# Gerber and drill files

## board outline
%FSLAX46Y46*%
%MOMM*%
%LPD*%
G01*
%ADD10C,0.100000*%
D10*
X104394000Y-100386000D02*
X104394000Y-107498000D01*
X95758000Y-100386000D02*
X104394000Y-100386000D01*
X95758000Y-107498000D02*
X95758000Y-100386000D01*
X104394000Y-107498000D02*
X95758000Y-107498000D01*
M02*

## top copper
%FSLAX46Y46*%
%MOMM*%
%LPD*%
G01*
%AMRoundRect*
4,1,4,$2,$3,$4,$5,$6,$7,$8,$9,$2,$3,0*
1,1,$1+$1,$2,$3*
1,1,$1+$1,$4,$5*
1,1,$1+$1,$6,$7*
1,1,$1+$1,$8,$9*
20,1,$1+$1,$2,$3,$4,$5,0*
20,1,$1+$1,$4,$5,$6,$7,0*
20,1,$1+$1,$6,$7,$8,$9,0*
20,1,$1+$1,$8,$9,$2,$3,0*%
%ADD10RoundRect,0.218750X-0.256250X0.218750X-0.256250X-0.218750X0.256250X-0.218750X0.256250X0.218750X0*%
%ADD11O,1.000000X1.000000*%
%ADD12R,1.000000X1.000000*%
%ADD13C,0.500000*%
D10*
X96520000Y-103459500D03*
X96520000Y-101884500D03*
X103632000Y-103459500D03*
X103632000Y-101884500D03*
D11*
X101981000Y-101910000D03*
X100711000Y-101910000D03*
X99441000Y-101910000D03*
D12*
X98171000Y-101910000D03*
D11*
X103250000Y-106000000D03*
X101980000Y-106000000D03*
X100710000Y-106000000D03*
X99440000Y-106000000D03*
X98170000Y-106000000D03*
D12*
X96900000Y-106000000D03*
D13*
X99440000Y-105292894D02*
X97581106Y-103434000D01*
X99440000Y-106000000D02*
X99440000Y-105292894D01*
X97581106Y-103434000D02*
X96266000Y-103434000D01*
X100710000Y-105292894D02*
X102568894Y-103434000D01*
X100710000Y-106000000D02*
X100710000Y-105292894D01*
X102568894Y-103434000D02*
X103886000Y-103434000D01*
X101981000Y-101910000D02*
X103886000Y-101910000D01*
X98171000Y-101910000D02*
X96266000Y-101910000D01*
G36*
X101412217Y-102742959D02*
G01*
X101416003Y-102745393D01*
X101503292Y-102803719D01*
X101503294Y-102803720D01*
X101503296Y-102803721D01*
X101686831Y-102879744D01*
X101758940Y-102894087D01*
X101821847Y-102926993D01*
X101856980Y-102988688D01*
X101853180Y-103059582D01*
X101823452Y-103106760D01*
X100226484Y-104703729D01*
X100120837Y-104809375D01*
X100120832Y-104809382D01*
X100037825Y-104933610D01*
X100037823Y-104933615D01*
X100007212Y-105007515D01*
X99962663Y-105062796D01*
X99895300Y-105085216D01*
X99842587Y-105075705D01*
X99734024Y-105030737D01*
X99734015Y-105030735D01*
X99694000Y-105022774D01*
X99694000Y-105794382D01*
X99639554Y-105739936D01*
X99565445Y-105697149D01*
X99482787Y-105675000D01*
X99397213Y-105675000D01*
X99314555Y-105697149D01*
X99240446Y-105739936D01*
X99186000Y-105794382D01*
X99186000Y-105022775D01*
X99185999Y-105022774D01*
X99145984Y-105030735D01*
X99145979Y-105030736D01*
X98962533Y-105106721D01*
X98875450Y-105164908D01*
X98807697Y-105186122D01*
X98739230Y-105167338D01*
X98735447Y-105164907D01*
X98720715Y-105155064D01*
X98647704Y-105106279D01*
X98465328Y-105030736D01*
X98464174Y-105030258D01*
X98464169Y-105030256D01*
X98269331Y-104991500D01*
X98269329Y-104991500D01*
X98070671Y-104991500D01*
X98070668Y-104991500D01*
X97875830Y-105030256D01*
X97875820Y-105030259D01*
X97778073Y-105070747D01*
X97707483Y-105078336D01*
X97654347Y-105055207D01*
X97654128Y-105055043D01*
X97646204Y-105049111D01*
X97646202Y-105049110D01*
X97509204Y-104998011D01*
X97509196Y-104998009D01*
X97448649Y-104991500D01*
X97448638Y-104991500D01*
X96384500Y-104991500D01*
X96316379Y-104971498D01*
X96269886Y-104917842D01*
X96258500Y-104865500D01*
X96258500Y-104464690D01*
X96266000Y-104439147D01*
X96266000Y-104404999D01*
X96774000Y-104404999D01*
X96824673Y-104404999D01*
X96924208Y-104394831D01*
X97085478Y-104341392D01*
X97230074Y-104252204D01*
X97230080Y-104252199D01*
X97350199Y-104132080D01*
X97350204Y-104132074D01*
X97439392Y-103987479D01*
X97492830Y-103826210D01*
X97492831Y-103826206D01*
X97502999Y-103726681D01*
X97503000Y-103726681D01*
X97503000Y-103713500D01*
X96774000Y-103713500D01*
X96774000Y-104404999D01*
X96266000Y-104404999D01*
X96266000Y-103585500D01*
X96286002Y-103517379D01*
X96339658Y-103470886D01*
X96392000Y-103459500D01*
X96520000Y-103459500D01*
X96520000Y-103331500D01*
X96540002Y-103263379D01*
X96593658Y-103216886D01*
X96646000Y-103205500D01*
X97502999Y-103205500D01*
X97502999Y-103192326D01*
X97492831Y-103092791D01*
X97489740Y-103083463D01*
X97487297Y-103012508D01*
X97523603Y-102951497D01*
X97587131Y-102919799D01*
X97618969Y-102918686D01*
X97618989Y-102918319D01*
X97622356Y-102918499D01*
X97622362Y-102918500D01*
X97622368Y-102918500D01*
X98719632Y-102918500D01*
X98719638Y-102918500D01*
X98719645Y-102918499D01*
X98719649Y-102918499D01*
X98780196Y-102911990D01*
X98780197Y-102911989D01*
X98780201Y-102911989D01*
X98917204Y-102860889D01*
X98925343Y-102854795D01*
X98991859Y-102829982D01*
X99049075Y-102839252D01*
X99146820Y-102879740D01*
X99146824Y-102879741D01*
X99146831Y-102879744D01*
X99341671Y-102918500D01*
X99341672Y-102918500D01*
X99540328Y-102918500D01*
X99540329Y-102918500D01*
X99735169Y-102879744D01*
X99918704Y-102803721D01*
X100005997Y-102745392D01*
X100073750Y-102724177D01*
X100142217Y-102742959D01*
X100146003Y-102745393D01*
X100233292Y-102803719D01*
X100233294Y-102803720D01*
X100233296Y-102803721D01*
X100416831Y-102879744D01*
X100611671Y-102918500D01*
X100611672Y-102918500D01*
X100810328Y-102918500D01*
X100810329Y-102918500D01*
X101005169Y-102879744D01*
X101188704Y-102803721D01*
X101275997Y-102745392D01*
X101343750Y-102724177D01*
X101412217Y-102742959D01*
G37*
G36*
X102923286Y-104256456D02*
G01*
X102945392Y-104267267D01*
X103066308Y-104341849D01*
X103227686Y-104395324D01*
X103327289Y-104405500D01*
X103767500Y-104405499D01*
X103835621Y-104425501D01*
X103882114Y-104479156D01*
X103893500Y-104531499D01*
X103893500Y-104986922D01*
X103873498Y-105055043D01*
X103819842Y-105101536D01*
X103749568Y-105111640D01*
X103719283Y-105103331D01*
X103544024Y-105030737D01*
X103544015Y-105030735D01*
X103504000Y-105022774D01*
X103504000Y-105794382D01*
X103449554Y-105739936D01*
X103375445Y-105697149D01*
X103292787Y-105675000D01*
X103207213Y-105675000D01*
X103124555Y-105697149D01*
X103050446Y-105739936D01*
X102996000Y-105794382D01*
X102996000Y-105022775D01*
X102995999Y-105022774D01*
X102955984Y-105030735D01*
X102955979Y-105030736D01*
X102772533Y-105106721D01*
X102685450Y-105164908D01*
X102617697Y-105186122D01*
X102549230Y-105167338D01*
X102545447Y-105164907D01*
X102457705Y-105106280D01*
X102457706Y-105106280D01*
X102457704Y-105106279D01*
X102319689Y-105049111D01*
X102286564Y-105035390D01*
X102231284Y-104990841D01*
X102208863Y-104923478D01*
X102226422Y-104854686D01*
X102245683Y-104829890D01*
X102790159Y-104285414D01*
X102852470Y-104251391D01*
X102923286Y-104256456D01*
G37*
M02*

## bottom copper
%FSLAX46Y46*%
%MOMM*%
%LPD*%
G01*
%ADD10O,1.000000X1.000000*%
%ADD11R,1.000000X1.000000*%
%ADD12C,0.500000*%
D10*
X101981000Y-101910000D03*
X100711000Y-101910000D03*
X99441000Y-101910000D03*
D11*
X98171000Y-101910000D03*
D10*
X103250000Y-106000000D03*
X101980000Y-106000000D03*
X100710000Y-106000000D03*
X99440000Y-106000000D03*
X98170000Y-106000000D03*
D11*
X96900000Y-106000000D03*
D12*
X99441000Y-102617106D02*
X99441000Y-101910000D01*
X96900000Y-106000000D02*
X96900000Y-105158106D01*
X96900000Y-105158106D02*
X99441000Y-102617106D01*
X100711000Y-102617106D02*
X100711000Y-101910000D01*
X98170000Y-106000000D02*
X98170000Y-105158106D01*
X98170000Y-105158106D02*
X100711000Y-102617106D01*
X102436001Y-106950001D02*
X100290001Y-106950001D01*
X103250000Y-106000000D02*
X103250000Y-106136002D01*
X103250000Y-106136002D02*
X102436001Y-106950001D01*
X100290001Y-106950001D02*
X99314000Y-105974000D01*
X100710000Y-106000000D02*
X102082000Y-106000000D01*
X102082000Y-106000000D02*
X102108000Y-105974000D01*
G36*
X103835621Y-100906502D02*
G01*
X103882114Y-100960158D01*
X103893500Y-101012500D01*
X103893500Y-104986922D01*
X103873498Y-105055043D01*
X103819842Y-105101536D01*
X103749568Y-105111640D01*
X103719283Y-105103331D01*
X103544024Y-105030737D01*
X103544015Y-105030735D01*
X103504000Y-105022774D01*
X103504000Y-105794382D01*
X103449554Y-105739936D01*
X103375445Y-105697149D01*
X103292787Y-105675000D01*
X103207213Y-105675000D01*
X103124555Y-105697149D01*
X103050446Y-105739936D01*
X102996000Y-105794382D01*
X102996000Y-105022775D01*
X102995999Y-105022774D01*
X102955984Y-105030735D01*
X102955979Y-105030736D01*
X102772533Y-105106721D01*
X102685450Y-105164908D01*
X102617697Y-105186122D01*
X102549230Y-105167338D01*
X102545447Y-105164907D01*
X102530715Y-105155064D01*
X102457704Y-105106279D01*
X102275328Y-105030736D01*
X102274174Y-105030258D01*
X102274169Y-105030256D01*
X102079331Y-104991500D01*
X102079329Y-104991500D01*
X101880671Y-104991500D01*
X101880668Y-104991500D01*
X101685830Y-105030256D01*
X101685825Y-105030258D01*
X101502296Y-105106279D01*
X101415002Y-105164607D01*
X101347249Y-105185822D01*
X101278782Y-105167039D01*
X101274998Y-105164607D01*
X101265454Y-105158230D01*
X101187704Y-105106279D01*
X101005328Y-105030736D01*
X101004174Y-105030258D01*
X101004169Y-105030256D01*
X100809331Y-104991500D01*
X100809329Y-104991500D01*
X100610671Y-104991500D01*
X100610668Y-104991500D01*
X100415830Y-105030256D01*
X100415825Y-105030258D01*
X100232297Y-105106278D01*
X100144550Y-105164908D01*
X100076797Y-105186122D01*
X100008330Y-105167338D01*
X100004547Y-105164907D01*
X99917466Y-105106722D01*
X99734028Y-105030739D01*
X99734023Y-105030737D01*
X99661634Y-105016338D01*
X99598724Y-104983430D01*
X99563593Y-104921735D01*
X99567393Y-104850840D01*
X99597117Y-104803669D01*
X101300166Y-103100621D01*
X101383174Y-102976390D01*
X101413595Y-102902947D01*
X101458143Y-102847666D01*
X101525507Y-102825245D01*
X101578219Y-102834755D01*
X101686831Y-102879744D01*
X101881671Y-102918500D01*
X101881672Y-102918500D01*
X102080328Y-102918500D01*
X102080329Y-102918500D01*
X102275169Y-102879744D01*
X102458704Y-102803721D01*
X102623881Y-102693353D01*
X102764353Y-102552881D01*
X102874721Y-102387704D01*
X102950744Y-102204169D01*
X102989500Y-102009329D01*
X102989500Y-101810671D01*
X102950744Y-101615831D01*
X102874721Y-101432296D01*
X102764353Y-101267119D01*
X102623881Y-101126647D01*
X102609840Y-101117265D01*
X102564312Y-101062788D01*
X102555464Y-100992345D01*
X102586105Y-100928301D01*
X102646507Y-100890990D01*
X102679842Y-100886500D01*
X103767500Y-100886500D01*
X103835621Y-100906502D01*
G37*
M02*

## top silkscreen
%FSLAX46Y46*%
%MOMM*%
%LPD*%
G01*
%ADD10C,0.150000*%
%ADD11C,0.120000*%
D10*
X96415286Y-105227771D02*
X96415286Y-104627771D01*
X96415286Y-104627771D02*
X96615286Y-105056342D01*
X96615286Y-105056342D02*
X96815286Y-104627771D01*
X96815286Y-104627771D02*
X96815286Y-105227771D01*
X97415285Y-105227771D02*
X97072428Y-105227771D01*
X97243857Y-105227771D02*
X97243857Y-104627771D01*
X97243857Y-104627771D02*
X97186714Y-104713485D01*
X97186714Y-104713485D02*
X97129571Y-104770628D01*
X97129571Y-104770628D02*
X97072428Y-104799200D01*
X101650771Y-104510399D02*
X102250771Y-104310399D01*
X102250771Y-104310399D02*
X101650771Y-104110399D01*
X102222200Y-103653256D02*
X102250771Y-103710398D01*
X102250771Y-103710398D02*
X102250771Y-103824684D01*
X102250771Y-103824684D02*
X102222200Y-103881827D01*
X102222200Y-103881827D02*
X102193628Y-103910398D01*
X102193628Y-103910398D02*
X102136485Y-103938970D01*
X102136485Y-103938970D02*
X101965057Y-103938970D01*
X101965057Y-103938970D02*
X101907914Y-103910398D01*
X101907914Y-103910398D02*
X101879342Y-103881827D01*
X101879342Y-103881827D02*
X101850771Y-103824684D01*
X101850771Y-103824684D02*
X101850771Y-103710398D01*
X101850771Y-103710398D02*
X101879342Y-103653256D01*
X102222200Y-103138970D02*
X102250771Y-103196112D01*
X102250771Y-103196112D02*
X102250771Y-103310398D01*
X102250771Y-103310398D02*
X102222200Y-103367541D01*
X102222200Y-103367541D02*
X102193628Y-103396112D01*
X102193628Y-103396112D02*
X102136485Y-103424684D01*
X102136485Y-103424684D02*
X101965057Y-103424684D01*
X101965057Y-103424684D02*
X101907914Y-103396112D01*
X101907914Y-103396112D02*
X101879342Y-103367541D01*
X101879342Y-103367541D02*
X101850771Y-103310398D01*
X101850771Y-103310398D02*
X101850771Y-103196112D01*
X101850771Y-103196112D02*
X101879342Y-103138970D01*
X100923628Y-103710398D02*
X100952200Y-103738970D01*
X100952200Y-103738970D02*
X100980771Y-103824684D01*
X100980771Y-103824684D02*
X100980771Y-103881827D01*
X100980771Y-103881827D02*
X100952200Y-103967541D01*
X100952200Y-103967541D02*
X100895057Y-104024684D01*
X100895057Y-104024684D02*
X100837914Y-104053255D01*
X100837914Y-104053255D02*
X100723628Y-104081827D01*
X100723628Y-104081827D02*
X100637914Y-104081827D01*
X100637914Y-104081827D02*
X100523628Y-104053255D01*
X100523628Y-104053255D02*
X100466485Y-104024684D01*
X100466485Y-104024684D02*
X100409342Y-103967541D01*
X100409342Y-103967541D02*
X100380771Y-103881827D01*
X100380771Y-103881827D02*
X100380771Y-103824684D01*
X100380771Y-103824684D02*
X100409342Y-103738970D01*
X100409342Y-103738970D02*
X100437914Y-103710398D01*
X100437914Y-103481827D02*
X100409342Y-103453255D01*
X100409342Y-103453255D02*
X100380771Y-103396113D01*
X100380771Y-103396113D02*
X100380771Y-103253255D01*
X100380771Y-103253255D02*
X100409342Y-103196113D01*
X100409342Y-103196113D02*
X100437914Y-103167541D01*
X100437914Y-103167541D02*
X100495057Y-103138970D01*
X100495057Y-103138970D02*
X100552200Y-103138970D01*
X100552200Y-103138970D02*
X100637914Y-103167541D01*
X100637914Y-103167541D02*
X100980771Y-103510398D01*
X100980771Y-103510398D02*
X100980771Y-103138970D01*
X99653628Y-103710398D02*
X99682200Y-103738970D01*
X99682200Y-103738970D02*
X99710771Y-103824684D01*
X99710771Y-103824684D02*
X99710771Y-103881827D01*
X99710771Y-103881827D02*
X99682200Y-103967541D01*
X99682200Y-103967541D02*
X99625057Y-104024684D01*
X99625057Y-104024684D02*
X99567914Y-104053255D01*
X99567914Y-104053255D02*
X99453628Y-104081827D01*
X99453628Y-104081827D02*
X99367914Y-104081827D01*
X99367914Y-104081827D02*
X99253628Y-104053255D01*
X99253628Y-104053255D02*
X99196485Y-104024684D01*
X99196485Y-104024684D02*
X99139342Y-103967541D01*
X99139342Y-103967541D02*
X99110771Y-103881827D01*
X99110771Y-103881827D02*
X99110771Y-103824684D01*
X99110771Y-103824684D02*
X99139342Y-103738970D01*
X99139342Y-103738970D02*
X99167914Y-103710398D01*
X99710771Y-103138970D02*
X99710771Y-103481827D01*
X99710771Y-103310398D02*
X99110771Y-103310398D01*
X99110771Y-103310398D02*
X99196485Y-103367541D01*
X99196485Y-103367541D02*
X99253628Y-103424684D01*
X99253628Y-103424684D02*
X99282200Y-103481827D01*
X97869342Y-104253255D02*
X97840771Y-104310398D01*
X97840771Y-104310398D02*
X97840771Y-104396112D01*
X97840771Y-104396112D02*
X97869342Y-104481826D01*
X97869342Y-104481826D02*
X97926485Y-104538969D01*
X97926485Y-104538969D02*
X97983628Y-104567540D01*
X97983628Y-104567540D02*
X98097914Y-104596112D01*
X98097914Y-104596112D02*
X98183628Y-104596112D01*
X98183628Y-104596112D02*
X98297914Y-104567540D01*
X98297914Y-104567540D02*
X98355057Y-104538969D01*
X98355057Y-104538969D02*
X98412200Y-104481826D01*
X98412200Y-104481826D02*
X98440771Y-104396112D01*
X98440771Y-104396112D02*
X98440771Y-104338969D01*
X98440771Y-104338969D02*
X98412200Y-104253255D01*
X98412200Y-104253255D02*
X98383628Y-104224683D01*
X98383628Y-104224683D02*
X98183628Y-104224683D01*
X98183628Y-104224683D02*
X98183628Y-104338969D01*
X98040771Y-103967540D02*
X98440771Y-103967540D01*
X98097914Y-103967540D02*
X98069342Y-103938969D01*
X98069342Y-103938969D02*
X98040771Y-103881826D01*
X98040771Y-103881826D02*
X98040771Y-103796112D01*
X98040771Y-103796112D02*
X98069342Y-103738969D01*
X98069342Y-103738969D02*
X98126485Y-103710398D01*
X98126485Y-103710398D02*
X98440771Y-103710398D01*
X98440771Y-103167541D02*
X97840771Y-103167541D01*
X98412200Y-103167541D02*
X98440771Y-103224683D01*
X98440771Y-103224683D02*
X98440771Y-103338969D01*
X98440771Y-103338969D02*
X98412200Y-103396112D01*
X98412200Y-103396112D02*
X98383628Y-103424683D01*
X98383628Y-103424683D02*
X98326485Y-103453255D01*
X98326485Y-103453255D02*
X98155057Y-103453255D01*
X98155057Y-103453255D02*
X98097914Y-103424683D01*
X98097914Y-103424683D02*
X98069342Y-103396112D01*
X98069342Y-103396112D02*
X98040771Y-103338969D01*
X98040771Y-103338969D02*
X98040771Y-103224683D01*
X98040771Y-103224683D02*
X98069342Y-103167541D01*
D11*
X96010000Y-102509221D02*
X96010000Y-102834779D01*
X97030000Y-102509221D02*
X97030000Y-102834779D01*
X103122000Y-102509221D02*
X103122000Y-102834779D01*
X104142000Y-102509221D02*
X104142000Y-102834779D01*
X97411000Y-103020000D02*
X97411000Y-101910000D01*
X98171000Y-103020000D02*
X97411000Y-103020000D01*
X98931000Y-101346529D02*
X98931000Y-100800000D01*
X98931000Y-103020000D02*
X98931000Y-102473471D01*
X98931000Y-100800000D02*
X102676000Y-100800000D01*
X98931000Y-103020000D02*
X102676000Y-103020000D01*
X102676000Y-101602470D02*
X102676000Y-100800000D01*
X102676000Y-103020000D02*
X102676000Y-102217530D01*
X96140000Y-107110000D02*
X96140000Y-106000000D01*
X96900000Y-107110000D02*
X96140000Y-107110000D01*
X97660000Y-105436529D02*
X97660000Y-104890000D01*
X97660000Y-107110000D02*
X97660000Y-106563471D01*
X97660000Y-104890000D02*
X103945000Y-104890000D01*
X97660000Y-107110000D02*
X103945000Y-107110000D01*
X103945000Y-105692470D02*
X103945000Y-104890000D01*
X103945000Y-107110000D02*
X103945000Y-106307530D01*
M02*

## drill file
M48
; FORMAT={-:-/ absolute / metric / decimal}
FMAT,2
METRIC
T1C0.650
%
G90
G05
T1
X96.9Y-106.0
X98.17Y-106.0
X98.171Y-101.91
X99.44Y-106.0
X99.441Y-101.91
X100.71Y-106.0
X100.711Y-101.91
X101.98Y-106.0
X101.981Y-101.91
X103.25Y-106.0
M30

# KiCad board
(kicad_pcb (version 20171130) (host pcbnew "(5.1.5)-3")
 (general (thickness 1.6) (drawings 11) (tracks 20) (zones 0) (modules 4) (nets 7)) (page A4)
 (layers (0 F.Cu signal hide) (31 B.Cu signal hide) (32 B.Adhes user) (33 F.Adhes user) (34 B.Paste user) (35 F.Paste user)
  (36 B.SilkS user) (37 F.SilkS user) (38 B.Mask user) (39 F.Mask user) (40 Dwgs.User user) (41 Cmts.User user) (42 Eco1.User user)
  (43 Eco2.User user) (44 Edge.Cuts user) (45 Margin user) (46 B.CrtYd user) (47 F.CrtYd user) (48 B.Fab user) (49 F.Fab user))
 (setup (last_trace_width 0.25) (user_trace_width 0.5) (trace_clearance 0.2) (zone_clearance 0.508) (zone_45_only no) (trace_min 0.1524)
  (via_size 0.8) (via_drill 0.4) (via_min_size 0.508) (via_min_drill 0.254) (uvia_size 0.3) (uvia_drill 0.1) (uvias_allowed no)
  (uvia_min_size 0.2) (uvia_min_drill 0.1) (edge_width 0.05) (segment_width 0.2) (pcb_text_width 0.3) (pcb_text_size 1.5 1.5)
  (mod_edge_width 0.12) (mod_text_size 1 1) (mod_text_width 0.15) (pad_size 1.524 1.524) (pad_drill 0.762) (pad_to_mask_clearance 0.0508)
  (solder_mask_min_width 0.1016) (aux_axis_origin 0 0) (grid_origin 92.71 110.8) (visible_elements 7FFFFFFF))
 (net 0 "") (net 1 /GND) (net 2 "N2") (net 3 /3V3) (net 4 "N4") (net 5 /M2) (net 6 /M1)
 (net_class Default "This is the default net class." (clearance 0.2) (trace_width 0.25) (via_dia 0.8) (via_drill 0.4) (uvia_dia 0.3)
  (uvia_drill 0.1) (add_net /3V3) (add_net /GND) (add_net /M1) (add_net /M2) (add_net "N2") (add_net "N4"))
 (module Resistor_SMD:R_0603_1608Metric (layer F.Cu) (at 96.52 102.672 270)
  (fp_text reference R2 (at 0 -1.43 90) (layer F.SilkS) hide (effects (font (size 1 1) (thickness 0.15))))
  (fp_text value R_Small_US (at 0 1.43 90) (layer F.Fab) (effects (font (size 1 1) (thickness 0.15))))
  (fp_line (start -0.162779 0.51) (end 0.162779 0.51) (layer F.SilkS) (width 0.12))
  (fp_line (start -0.162779 -0.51) (end 0.162779 -0.51) (layer F.SilkS) (width 0.12))
  (pad 2 smd roundrect (at 0.7875 0 270) (size 0.875 0.95) (layers F.Cu F.Paste F.Mask) (roundrect_rratio 0.25) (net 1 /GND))
  (pad 1 smd roundrect (at -0.7875 0 270) (size 0.875 0.95) (layers F.Cu F.Paste F.Mask) (roundrect_rratio 0.25) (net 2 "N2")))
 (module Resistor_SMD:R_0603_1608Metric (layer F.Cu) (at 103.632 102.672 270)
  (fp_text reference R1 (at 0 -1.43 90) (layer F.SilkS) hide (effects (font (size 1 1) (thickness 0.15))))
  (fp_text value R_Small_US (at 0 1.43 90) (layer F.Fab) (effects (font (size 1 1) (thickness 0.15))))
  (fp_line (start -0.162779 0.51) (end 0.162779 0.51) (layer F.SilkS) (width 0.12))
  (fp_line (start -0.162779 -0.51) (end 0.162779 -0.51) (layer F.SilkS) (width 0.12))
  (pad 2 smd roundrect (at 0.7875 0 270) (size 0.875 0.95) (layers F.Cu F.Paste F.Mask) (roundrect_rratio 0.25) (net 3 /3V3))
  (pad 1 smd roundrect (at -0.7875 0 270) (size 0.875 0.95) (layers F.Cu F.Paste F.Mask) (roundrect_rratio 0.25) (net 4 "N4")))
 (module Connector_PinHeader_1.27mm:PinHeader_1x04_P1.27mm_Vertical (layer F.Cu) (at 98.171 101.91 90)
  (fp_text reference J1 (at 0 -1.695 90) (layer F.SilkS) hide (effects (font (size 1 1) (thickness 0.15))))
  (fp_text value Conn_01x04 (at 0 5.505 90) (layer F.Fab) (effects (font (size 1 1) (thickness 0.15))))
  (fp_line (start -1.11 -0.76) (end 0 -0.76) (layer F.SilkS) (width 0.12))
  (fp_line (start -1.11 0) (end -1.11 -0.76) (layer F.SilkS) (width 0.12))
  (fp_line (start 0.563471 0.76) (end 1.11 0.76) (layer F.SilkS) (width 0.12))
  (fp_line (start -1.11 0.76) (end -0.563471 0.76) (layer F.SilkS) (width 0.12))
  (fp_line (start 1.11 0.76) (end 1.11 4.505) (layer F.SilkS) (width 0.12))
  (fp_line (start -1.11 0.76) (end -1.11 4.505) (layer F.SilkS) (width 0.12))
  (fp_line (start 0.30753 4.505) (end 1.11 4.505) (layer F.SilkS) (width 0.12))
  (fp_line (start -1.11 4.505) (end -0.30753 4.505) (layer F.SilkS) (width 0.12))
  (pad 4 thru_hole oval (at 0 3.81 90) (size 1 1) (drill 0.65) (layers *.Cu *.Mask) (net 4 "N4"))
  (pad 3 thru_hole oval (at 0 2.54 90) (size 1 1) (drill 0.65) (layers *.Cu *.Mask) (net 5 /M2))
  (pad 2 thru_hole oval (at 0 1.27 90) (size 1 1) (drill 0.65) (layers *.Cu *.Mask) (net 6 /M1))
  (pad 1 thru_hole rect (at 0 0 90) (size 1 1) (drill 0.65) (layers *.Cu *.Mask) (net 2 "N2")))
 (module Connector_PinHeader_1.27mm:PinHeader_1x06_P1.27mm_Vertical (layer F.Cu) (at 96.9 106 90)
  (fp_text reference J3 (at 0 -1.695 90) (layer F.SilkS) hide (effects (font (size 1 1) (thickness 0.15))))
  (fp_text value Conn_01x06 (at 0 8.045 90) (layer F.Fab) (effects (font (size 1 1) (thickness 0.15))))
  (fp_line (start -1.11 -0.76) (end 0 -0.76) (layer F.SilkS) (width 0.12))
  (fp_line (start -1.11 0) (end -1.11 -0.76) (layer F.SilkS) (width 0.12))
  (fp_line (start 0.563471 0.76) (end 1.11 0.76) (layer F.SilkS) (width 0.12))
  (fp_line (start -1.11 0.76) (end -0.563471 0.76) (layer F.SilkS) (width 0.12))
  (fp_line (start 1.11 0.76) (end 1.11 7.045) (layer F.SilkS) (width 0.12))
  (fp_line (start -1.11 0.76) (end -1.11 7.045) (layer F.SilkS) (width 0.12))
  (fp_line (start 0.30753 7.045) (end 1.11 7.045) (layer F.SilkS) (width 0.12))
  (fp_line (start -1.11 7.045) (end -0.30753 7.045) (layer F.SilkS) (width 0.12))
  (pad 6 thru_hole oval (at 0 6.35 90) (size 1 1) (drill 0.65) (layers *.Cu *.Mask) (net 1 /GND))
  (pad 5 thru_hole oval (at 0 5.08 90) (size 1 1) (drill 0.65) (layers *.Cu *.Mask) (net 3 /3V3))
  (pad 4 thru_hole oval (at 0 3.81 90) (size 1 1) (drill 0.65) (layers *.Cu *.Mask) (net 3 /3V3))
  (pad 3 thru_hole oval (at 0 2.54 90) (size 1 1) (drill 0.65) (layers *.Cu *.Mask) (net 1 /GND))
  (pad 2 thru_hole oval (at 0 1.27 90) (size 1 1) (drill 0.65) (layers *.Cu *.Mask) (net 5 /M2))
  (pad 1 thru_hole rect (at 0 0 90) (size 1 1) (drill 0.65) (layers *.Cu *.Mask) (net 6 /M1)))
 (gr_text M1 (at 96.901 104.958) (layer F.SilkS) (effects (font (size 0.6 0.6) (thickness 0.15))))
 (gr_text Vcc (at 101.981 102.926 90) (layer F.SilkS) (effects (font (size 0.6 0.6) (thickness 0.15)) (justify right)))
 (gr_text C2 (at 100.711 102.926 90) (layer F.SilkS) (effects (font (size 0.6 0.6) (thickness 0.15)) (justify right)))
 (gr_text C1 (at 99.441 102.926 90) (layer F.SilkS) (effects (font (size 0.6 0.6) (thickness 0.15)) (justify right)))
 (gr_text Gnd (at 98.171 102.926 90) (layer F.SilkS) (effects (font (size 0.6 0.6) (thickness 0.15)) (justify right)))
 (gr_line (start 104.394 100.386) (end 104.394 107.498) (layer Edge.Cuts) (width 0.1))
 (gr_line (start 95.758 100.386) (end 104.394 100.386) (layer Edge.Cuts) (width 0.1))
 (gr_line (start 95.758 107.498) (end 95.758 100.386) (layer Edge.Cuts) (width 0.1))
 (gr_line (start 104.394 107.498) (end 95.758 107.498) (layer Edge.Cuts) (width 0.1))
 (segment (start 99.441 102.617106) (end 99.441 101.91) (width 0.5) (layer B.Cu) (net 6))
 (segment (start 96.9 106) (end 96.9 105.158106) (width 0.5) (layer B.Cu) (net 6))
 (segment (start 96.9 105.158106) (end 99.441 102.617106) (width 0.5) (layer B.Cu) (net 6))
 (segment (start 100.711 102.617106) (end 100.711 101.91) (width 0.5) (layer B.Cu) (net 5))
 (segment (start 98.17 106) (end 98.17 105.158106) (width 0.5) (layer B.Cu) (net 5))
 (segment (start 98.17 105.158106) (end 100.711 102.617106) (width 0.5) (layer B.Cu) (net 5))
 (segment (start 102.436001 106.950001) (end 100.290001 106.950001) (width 0.5) (layer B.Cu) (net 1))
 (segment (start 103.25 106) (end 103.25 106.136002) (width 0.5) (layer B.Cu) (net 1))
 (segment (start 103.25 106.136002) (end 102.436001 106.950001) (width 0.5) (layer B.Cu) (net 1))
 (segment (start 100.290001 106.950001) (end 99.314 105.974) (width 0.5) (layer B.Cu) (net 1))
 (segment (start 99.44 105.292894) (end 97.581106 103.434) (width 0.5) (layer F.Cu) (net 1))
 (segment (start 99.44 106) (end 99.44 105.292894) (width 0.5) (layer F.Cu) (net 1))
 (segment (start 97.581106 103.434) (end 96.266 103.434) (width 0.5) (layer F.Cu) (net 1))
 (segment (start 100.71 105.292894) (end 102.568894 103.434) (width 0.5) (layer F.Cu) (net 3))
 (segment (start 100.71 106) (end 100.71 105.292894) (width 0.5) (layer F.Cu) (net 3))
 (segment (start 102.568894 103.434) (end 103.886 103.434) (width 0.5) (layer F.Cu) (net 3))
 (segment (start 100.71 106) (end 102.082 106) (width 0.5) (layer B.Cu) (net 3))
 (segment (start 102.082 106) (end 102.108 105.974) (width 0.5) (layer B.Cu) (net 3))
 (segment (start 101.981 101.91) (end 103.886 101.91) (width 0.5) (layer F.Cu) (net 4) (status 30))
 (segment (start 98.171 101.91) (end 96.266 101.91) (width 0.5) (layer F.Cu) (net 2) (status 30))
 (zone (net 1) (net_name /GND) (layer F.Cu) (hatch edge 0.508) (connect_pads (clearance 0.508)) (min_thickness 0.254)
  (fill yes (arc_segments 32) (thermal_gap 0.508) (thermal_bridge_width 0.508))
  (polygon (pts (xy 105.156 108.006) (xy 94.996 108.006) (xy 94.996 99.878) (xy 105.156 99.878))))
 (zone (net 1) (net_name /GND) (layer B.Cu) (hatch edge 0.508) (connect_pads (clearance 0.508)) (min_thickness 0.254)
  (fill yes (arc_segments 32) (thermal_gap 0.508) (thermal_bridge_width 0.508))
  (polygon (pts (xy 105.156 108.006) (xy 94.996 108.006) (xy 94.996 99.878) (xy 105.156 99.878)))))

